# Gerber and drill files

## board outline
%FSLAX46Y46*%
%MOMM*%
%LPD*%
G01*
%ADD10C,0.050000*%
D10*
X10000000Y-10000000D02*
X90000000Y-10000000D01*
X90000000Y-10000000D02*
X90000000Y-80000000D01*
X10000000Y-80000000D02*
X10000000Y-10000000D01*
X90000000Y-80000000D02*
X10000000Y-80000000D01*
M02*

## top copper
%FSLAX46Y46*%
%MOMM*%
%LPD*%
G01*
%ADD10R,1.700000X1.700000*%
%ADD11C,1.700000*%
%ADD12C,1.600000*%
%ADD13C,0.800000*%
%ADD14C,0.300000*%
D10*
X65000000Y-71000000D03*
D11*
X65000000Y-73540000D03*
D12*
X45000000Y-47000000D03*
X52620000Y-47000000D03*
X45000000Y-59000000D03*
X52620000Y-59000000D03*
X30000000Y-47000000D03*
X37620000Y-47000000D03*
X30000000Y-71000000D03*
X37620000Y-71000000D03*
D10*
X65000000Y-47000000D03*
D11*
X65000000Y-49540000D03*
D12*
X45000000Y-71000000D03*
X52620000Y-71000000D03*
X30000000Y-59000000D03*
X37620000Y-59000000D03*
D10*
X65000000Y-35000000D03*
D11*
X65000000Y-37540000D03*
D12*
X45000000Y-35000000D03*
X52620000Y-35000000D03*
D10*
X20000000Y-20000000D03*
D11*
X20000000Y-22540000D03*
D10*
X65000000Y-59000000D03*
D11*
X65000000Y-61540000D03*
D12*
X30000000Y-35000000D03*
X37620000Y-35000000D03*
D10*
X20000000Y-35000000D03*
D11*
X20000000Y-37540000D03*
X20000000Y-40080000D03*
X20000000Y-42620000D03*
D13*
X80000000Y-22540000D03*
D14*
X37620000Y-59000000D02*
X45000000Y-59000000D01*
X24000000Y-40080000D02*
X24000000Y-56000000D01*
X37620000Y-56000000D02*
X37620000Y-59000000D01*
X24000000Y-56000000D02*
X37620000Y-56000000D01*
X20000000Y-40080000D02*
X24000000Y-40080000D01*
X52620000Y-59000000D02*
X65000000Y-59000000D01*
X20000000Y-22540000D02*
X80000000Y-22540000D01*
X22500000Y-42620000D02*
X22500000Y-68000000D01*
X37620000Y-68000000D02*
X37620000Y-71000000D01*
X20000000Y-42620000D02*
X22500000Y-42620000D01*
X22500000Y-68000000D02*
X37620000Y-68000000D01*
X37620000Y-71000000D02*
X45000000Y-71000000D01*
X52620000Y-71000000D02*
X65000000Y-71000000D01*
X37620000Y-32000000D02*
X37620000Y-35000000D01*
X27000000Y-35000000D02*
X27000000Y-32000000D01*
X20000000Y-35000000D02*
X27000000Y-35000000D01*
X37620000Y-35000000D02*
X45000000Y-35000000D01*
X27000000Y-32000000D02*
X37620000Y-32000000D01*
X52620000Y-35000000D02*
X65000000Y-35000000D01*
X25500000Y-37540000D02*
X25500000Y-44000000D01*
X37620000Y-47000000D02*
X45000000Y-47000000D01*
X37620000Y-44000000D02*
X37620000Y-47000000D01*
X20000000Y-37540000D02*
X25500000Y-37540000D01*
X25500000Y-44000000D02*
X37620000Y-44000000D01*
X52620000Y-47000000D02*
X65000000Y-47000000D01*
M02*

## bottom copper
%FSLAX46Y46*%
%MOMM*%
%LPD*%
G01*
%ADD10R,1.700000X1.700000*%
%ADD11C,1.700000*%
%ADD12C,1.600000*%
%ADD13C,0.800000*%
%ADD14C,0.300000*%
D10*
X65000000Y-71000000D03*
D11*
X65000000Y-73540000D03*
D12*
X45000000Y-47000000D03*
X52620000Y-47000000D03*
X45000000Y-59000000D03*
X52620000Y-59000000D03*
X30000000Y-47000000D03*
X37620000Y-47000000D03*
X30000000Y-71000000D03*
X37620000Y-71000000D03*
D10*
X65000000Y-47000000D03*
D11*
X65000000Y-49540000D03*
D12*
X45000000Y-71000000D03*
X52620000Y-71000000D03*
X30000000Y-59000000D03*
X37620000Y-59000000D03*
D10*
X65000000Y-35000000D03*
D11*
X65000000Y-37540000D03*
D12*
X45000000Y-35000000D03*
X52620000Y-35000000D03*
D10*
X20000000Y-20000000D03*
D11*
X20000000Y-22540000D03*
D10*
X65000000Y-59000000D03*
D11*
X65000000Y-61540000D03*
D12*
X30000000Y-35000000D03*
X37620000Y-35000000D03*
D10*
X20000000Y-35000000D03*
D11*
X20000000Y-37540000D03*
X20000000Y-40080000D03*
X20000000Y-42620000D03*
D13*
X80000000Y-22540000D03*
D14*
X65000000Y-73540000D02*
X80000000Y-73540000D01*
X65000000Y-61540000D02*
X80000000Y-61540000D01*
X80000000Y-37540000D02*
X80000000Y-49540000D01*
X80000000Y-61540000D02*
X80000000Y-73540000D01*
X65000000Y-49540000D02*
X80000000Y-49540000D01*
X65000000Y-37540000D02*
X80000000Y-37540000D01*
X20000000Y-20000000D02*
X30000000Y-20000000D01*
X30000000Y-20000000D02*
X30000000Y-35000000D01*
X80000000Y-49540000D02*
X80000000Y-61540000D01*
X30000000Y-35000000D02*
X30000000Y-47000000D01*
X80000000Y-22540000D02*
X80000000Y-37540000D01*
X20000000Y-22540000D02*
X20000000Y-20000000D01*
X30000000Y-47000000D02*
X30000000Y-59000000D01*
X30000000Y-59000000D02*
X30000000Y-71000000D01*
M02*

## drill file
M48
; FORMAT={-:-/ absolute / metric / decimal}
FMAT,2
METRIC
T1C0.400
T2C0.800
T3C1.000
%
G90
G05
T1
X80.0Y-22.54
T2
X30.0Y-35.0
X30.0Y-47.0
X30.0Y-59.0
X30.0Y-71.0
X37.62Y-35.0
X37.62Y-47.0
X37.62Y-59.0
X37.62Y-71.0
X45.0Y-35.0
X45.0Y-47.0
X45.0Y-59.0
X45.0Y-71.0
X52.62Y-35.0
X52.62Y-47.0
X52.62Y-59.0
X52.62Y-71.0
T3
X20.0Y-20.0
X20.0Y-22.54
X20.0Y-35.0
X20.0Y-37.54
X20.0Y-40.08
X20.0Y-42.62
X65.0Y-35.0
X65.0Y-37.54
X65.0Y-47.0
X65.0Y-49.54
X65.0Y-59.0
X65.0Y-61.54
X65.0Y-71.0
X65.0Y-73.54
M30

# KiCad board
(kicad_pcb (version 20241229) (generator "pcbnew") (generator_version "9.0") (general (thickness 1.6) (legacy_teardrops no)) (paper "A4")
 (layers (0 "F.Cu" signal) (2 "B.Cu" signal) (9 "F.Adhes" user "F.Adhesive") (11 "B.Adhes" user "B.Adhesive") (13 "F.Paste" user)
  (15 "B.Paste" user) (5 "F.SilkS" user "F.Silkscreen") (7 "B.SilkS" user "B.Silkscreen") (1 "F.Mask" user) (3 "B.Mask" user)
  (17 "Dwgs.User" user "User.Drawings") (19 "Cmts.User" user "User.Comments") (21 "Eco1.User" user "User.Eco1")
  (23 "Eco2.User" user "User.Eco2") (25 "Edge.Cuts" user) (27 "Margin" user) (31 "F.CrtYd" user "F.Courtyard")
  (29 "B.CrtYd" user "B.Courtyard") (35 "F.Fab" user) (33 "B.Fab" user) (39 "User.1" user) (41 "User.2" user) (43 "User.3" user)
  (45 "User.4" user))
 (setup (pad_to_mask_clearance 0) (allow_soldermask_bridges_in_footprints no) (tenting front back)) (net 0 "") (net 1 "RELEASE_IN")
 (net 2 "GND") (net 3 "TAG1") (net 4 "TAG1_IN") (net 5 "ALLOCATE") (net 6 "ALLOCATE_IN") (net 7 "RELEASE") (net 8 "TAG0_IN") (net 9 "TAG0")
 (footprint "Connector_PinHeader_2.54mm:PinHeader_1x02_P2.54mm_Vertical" (layer "F.Cu") (at 65 71)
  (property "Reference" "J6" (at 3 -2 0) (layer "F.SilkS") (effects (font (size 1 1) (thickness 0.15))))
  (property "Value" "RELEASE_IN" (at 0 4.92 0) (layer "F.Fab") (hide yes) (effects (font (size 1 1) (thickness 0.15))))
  (pad "1" thru_hole rect (at 0 0) (size 1.7 1.7) (drill 1) (layers "*.Cu" "*.Mask") (remove_unused_layers no) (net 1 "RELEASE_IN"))
  (pad "2" thru_hole circle (at 0 2.54) (size 1.7 1.7) (drill 1) (layers "*.Cu" "*.Mask") (remove_unused_layers no) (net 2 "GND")))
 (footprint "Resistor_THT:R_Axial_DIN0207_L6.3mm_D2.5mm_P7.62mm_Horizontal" (layer "F.Cu") (at 45 47)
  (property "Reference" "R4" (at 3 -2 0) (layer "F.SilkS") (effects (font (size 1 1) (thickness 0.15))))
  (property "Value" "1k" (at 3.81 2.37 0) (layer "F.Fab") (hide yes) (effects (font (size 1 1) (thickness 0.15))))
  (pad "1" thru_hole circle (at 0 0) (size 1.6 1.6) (drill 0.8) (layers "*.Cu" "*.Mask") (remove_unused_layers no) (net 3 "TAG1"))
  (pad "2" thru_hole circle (at 7.62 0) (size 1.6 1.6) (drill 0.8) (layers "*.Cu" "*.Mask") (remove_unused_layers no) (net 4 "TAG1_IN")))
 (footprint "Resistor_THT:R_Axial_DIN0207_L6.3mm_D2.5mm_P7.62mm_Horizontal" (layer "F.Cu") (at 45 59)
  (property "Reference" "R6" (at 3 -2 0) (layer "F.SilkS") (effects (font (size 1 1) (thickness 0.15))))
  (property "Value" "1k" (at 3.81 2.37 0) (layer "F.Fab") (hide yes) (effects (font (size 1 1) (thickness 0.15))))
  (pad "1" thru_hole circle (at 0 0) (size 1.6 1.6) (drill 0.8) (layers "*.Cu" "*.Mask") (remove_unused_layers no) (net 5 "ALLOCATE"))
  (pad "2" thru_hole circle (at 7.62 0) (size 1.6 1.6) (drill 0.8) (layers "*.Cu" "*.Mask") (remove_unused_layers no) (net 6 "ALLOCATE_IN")))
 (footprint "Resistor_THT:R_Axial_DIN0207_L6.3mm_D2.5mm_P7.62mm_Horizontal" (layer "F.Cu") (at 30 47)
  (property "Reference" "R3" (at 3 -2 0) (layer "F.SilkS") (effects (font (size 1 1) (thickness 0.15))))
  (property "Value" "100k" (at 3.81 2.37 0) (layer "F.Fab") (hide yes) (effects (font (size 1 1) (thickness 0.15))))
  (pad "1" thru_hole circle (at 0 0) (size 1.6 1.6) (drill 0.8) (layers "*.Cu" "*.Mask") (remove_unused_layers no) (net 2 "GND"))
  (pad "2" thru_hole circle (at 7.62 0) (size 1.6 1.6) (drill 0.8) (layers "*.Cu" "*.Mask") (remove_unused_layers no) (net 3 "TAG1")))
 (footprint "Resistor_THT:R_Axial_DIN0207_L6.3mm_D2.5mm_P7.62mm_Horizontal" (layer "F.Cu") (at 30 71)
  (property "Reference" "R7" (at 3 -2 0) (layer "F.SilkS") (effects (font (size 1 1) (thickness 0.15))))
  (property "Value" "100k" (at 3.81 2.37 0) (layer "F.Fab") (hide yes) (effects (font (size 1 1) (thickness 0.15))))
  (pad "1" thru_hole circle (at 0 0) (size 1.6 1.6) (drill 0.8) (layers "*.Cu" "*.Mask") (remove_unused_layers no) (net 2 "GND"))
  (pad "2" thru_hole circle (at 7.62 0) (size 1.6 1.6) (drill 0.8) (layers "*.Cu" "*.Mask") (remove_unused_layers no) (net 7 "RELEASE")))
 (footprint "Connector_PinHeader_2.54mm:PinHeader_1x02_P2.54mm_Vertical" (layer "F.Cu") (at 65 47)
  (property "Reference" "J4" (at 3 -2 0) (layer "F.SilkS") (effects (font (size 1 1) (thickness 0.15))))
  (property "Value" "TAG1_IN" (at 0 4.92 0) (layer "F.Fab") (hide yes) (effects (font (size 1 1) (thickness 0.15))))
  (pad "1" thru_hole rect (at 0 0) (size 1.7 1.7) (drill 1) (layers "*.Cu" "*.Mask") (remove_unused_layers no) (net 4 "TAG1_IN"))
  (pad "2" thru_hole circle (at 0 2.54) (size 1.7 1.7) (drill 1) (layers "*.Cu" "*.Mask") (remove_unused_layers no) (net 2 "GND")))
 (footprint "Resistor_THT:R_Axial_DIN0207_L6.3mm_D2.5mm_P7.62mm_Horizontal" (layer "F.Cu") (at 45 71)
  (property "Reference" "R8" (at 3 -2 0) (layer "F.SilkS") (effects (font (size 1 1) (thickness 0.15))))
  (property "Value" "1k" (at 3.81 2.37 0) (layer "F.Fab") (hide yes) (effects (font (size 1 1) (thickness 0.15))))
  (pad "1" thru_hole circle (at 0 0) (size 1.6 1.6) (drill 0.8) (layers "*.Cu" "*.Mask") (remove_unused_layers no) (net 7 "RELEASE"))
  (pad "2" thru_hole circle (at 7.62 0) (size 1.6 1.6) (drill 0.8) (layers "*.Cu" "*.Mask") (remove_unused_layers no) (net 1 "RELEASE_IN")))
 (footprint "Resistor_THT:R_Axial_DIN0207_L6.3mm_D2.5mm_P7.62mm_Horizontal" (layer "F.Cu") (at 30 59)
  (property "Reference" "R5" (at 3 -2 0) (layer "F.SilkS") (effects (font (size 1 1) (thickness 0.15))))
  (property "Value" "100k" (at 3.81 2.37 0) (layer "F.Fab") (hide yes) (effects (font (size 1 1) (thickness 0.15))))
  (pad "1" thru_hole circle (at 0 0) (size 1.6 1.6) (drill 0.8) (layers "*.Cu" "*.Mask") (remove_unused_layers no) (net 2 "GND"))
  (pad "2" thru_hole circle (at 7.62 0) (size 1.6 1.6) (drill 0.8) (layers "*.Cu" "*.Mask") (remove_unused_layers no) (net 5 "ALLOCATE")))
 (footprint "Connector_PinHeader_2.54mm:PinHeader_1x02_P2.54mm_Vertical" (layer "F.Cu") (at 65 35)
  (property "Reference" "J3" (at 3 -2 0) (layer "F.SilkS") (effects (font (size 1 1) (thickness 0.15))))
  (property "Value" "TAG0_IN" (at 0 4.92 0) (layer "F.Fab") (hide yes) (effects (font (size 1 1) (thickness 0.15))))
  (pad "1" thru_hole rect (at 0 0) (size 1.7 1.7) (drill 1) (layers "*.Cu" "*.Mask") (remove_unused_layers no) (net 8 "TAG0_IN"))
  (pad "2" thru_hole circle (at 0 2.54) (size 1.7 1.7) (drill 1) (layers "*.Cu" "*.Mask") (remove_unused_layers no) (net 2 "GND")))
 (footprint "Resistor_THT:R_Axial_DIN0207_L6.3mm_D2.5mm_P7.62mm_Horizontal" (layer "F.Cu") (at 45 35)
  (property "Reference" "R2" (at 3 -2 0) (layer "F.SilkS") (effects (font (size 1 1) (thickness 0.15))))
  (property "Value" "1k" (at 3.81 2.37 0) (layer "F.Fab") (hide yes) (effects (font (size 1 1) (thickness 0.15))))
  (pad "1" thru_hole circle (at 0 0) (size 1.6 1.6) (drill 0.8) (layers "*.Cu" "*.Mask") (remove_unused_layers no) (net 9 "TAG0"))
  (pad "2" thru_hole circle (at 7.62 0) (size 1.6 1.6) (drill 0.8) (layers "*.Cu" "*.Mask") (remove_unused_layers no) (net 8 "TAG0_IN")))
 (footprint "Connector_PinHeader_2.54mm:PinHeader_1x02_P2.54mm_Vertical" (layer "F.Cu") (at 20 20)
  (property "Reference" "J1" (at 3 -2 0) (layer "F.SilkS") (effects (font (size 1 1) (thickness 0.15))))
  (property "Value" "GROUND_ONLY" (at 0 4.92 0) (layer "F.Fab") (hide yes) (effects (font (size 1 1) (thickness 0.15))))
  (pad "1" thru_hole rect (at 0 0) (size 1.7 1.7) (drill 1) (layers "*.Cu" "*.Mask") (remove_unused_layers no) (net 2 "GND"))
  (pad "2" thru_hole circle (at 0 2.54) (size 1.7 1.7) (drill 1) (layers "*.Cu" "*.Mask") (remove_unused_layers no) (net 2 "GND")))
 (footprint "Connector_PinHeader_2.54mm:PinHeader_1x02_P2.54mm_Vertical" (layer "F.Cu") (at 65 59)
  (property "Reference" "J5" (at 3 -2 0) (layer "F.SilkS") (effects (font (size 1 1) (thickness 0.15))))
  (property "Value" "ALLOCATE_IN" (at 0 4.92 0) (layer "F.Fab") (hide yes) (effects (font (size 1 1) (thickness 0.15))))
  (pad "1" thru_hole rect (at 0 0) (size 1.7 1.7) (drill 1) (layers "*.Cu" "*.Mask") (remove_unused_layers no) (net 6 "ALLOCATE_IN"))
  (pad "2" thru_hole circle (at 0 2.54) (size 1.7 1.7) (drill 1) (layers "*.Cu" "*.Mask") (remove_unused_layers no) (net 2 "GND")))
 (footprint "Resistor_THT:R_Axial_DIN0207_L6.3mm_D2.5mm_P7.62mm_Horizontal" (layer "F.Cu") (at 30 35)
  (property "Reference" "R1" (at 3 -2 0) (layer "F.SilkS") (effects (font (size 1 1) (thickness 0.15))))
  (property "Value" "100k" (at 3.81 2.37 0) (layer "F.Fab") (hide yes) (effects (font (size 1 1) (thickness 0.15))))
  (pad "1" thru_hole circle (at 0 0) (size 1.6 1.6) (drill 0.8) (layers "*.Cu" "*.Mask") (remove_unused_layers no) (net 2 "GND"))
  (pad "2" thru_hole circle (at 7.62 0) (size 1.6 1.6) (drill 0.8) (layers "*.Cu" "*.Mask") (remove_unused_layers no) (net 9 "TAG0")))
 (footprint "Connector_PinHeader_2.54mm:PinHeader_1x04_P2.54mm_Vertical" (layer "F.Cu") (at 20 35)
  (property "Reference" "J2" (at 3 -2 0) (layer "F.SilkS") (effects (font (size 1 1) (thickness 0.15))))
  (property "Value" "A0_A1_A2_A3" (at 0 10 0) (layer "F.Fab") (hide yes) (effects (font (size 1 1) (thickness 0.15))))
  (pad "1" thru_hole rect (at 0 0) (size 1.7 1.7) (drill 1) (layers "*.Cu" "*.Mask") (remove_unused_layers no) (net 9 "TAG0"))
  (pad "2" thru_hole circle (at 0 2.54) (size 1.7 1.7) (drill 1) (layers "*.Cu" "*.Mask") (remove_unused_layers no) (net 3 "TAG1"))
  (pad "3" thru_hole circle (at 0 5.08) (size 1.7 1.7) (drill 1) (layers "*.Cu" "*.Mask") (remove_unused_layers no) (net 5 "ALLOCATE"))
  (pad "4" thru_hole circle (at 0 7.62) (size 1.7 1.7) (drill 1) (layers "*.Cu" "*.Mask") (remove_unused_layers no) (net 7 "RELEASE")))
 (gr_line (start 10 10) (end 90 10) (stroke (width 0.05) (type default)) (layer "Edge.Cuts"))
 (gr_line (start 90 10) (end 90 80) (stroke (width 0.05) (type default)) (layer "Edge.Cuts"))
 (gr_line (start 10 80) (end 10 10) (stroke (width 0.05) (type default)) (layer "Edge.Cuts"))
 (gr_line (start 90 80) (end 10 80) (stroke (width 0.05) (type default)) (layer "Edge.Cuts"))
 (segment (start 37.62 59) (end 45 59) (width 0.3) (layer "F.Cu") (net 5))
 (segment (start 24 40.08) (end 24 56) (width 0.3) (layer "F.Cu") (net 5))
 (segment (start 37.62 56) (end 37.62 59) (width 0.3) (layer "F.Cu") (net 5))
 (segment (start 24 56) (end 37.62 56) (width 0.3) (layer "F.Cu") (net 5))
 (segment (start 20 40.08) (end 24 40.08) (width 0.3) (layer "F.Cu") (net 5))
 (segment (start 52.62 59) (end 65 59) (width 0.3) (layer "F.Cu") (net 6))
 (segment (start 20 22.54) (end 80 22.54) (width 0.3) (layer "F.Cu") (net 2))
 (via (at 80 22.54) (size 0.8) (drill 0.4) (layers "F.Cu" "B.Cu") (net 2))
 (segment (start 65 73.54) (end 80 73.54) (width 0.3) (layer "B.Cu") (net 2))
 (segment (start 65 61.54) (end 80 61.54) (width 0.3) (layer "B.Cu") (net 2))
 (segment (start 80 37.54) (end 80 49.54) (width 0.3) (layer "B.Cu") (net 2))
 (segment (start 80 61.54) (end 80 73.54) (width 0.3) (layer "B.Cu") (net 2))
 (segment (start 65 49.54) (end 80 49.54) (width 0.3) (layer "B.Cu") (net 2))
 (segment (start 65 37.54) (end 80 37.54) (width 0.3) (layer "B.Cu") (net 2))
 (segment (start 20 20) (end 30 20) (width 0.3) (layer "B.Cu") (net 2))
 (segment (start 30 20) (end 30 35) (width 0.3) (layer "B.Cu") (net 2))
 (segment (start 80 49.54) (end 80 61.54) (width 0.3) (layer "B.Cu") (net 2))
 (segment (start 30 35) (end 30 47) (width 0.3) (layer "B.Cu") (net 2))
 (segment (start 80 22.54) (end 80 37.54) (width 0.3) (layer "B.Cu") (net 2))
 (segment (start 20 22.54) (end 20 20) (width 0.3) (layer "B.Cu") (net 2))
 (segment (start 30 47) (end 30 59) (width 0.3) (layer "B.Cu") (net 2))
 (segment (start 30 59) (end 30 71) (width 0.3) (layer "B.Cu") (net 2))
 (segment (start 22.5 42.62) (end 22.5 68) (width 0.3) (layer "F.Cu") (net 7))
 (segment (start 37.62 68) (end 37.62 71) (width 0.3) (layer "F.Cu") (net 7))
 (segment (start 20 42.62) (end 22.5 42.62) (width 0.3) (layer "F.Cu") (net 7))
 (segment (start 22.5 68) (end 37.62 68) (width 0.3) (layer "F.Cu") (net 7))
 (segment (start 37.62 71) (end 45 71) (width 0.3) (layer "F.Cu") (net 7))
 (segment (start 52.62 71) (end 65 71) (width 0.3) (layer "F.Cu") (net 1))
 (segment (start 37.62 32) (end 37.62 35) (width 0.3) (layer "F.Cu") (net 9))
 (segment (start 27 35) (end 27 32) (width 0.3) (layer "F.Cu") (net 9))
 (segment (start 20 35) (end 27 35) (width 0.3) (layer "F.Cu") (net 9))
 (segment (start 37.62 35) (end 45 35) (width 0.3) (layer "F.Cu") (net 9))
 (segment (start 27 32) (end 37.62 32) (width 0.3) (layer "F.Cu") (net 9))
 (segment (start 52.62 35) (end 65 35) (width 0.3) (layer "F.Cu") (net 8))
 (segment (start 25.5 37.54) (end 25.5 44) (width 0.3) (layer "F.Cu") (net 3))
 (segment (start 37.62 47) (end 45 47) (width 0.3) (layer "F.Cu") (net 3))
 (segment (start 37.62 44) (end 37.62 47) (width 0.3) (layer "F.Cu") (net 3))
 (segment (start 20 37.54) (end 25.5 37.54) (width 0.3) (layer "F.Cu") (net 3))
 (segment (start 25.5 44) (end 37.62 44) (width 0.3) (layer "F.Cu") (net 3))
 (segment (start 52.62 47) (end 65 47) (width 0.3) (layer "F.Cu") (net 4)))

